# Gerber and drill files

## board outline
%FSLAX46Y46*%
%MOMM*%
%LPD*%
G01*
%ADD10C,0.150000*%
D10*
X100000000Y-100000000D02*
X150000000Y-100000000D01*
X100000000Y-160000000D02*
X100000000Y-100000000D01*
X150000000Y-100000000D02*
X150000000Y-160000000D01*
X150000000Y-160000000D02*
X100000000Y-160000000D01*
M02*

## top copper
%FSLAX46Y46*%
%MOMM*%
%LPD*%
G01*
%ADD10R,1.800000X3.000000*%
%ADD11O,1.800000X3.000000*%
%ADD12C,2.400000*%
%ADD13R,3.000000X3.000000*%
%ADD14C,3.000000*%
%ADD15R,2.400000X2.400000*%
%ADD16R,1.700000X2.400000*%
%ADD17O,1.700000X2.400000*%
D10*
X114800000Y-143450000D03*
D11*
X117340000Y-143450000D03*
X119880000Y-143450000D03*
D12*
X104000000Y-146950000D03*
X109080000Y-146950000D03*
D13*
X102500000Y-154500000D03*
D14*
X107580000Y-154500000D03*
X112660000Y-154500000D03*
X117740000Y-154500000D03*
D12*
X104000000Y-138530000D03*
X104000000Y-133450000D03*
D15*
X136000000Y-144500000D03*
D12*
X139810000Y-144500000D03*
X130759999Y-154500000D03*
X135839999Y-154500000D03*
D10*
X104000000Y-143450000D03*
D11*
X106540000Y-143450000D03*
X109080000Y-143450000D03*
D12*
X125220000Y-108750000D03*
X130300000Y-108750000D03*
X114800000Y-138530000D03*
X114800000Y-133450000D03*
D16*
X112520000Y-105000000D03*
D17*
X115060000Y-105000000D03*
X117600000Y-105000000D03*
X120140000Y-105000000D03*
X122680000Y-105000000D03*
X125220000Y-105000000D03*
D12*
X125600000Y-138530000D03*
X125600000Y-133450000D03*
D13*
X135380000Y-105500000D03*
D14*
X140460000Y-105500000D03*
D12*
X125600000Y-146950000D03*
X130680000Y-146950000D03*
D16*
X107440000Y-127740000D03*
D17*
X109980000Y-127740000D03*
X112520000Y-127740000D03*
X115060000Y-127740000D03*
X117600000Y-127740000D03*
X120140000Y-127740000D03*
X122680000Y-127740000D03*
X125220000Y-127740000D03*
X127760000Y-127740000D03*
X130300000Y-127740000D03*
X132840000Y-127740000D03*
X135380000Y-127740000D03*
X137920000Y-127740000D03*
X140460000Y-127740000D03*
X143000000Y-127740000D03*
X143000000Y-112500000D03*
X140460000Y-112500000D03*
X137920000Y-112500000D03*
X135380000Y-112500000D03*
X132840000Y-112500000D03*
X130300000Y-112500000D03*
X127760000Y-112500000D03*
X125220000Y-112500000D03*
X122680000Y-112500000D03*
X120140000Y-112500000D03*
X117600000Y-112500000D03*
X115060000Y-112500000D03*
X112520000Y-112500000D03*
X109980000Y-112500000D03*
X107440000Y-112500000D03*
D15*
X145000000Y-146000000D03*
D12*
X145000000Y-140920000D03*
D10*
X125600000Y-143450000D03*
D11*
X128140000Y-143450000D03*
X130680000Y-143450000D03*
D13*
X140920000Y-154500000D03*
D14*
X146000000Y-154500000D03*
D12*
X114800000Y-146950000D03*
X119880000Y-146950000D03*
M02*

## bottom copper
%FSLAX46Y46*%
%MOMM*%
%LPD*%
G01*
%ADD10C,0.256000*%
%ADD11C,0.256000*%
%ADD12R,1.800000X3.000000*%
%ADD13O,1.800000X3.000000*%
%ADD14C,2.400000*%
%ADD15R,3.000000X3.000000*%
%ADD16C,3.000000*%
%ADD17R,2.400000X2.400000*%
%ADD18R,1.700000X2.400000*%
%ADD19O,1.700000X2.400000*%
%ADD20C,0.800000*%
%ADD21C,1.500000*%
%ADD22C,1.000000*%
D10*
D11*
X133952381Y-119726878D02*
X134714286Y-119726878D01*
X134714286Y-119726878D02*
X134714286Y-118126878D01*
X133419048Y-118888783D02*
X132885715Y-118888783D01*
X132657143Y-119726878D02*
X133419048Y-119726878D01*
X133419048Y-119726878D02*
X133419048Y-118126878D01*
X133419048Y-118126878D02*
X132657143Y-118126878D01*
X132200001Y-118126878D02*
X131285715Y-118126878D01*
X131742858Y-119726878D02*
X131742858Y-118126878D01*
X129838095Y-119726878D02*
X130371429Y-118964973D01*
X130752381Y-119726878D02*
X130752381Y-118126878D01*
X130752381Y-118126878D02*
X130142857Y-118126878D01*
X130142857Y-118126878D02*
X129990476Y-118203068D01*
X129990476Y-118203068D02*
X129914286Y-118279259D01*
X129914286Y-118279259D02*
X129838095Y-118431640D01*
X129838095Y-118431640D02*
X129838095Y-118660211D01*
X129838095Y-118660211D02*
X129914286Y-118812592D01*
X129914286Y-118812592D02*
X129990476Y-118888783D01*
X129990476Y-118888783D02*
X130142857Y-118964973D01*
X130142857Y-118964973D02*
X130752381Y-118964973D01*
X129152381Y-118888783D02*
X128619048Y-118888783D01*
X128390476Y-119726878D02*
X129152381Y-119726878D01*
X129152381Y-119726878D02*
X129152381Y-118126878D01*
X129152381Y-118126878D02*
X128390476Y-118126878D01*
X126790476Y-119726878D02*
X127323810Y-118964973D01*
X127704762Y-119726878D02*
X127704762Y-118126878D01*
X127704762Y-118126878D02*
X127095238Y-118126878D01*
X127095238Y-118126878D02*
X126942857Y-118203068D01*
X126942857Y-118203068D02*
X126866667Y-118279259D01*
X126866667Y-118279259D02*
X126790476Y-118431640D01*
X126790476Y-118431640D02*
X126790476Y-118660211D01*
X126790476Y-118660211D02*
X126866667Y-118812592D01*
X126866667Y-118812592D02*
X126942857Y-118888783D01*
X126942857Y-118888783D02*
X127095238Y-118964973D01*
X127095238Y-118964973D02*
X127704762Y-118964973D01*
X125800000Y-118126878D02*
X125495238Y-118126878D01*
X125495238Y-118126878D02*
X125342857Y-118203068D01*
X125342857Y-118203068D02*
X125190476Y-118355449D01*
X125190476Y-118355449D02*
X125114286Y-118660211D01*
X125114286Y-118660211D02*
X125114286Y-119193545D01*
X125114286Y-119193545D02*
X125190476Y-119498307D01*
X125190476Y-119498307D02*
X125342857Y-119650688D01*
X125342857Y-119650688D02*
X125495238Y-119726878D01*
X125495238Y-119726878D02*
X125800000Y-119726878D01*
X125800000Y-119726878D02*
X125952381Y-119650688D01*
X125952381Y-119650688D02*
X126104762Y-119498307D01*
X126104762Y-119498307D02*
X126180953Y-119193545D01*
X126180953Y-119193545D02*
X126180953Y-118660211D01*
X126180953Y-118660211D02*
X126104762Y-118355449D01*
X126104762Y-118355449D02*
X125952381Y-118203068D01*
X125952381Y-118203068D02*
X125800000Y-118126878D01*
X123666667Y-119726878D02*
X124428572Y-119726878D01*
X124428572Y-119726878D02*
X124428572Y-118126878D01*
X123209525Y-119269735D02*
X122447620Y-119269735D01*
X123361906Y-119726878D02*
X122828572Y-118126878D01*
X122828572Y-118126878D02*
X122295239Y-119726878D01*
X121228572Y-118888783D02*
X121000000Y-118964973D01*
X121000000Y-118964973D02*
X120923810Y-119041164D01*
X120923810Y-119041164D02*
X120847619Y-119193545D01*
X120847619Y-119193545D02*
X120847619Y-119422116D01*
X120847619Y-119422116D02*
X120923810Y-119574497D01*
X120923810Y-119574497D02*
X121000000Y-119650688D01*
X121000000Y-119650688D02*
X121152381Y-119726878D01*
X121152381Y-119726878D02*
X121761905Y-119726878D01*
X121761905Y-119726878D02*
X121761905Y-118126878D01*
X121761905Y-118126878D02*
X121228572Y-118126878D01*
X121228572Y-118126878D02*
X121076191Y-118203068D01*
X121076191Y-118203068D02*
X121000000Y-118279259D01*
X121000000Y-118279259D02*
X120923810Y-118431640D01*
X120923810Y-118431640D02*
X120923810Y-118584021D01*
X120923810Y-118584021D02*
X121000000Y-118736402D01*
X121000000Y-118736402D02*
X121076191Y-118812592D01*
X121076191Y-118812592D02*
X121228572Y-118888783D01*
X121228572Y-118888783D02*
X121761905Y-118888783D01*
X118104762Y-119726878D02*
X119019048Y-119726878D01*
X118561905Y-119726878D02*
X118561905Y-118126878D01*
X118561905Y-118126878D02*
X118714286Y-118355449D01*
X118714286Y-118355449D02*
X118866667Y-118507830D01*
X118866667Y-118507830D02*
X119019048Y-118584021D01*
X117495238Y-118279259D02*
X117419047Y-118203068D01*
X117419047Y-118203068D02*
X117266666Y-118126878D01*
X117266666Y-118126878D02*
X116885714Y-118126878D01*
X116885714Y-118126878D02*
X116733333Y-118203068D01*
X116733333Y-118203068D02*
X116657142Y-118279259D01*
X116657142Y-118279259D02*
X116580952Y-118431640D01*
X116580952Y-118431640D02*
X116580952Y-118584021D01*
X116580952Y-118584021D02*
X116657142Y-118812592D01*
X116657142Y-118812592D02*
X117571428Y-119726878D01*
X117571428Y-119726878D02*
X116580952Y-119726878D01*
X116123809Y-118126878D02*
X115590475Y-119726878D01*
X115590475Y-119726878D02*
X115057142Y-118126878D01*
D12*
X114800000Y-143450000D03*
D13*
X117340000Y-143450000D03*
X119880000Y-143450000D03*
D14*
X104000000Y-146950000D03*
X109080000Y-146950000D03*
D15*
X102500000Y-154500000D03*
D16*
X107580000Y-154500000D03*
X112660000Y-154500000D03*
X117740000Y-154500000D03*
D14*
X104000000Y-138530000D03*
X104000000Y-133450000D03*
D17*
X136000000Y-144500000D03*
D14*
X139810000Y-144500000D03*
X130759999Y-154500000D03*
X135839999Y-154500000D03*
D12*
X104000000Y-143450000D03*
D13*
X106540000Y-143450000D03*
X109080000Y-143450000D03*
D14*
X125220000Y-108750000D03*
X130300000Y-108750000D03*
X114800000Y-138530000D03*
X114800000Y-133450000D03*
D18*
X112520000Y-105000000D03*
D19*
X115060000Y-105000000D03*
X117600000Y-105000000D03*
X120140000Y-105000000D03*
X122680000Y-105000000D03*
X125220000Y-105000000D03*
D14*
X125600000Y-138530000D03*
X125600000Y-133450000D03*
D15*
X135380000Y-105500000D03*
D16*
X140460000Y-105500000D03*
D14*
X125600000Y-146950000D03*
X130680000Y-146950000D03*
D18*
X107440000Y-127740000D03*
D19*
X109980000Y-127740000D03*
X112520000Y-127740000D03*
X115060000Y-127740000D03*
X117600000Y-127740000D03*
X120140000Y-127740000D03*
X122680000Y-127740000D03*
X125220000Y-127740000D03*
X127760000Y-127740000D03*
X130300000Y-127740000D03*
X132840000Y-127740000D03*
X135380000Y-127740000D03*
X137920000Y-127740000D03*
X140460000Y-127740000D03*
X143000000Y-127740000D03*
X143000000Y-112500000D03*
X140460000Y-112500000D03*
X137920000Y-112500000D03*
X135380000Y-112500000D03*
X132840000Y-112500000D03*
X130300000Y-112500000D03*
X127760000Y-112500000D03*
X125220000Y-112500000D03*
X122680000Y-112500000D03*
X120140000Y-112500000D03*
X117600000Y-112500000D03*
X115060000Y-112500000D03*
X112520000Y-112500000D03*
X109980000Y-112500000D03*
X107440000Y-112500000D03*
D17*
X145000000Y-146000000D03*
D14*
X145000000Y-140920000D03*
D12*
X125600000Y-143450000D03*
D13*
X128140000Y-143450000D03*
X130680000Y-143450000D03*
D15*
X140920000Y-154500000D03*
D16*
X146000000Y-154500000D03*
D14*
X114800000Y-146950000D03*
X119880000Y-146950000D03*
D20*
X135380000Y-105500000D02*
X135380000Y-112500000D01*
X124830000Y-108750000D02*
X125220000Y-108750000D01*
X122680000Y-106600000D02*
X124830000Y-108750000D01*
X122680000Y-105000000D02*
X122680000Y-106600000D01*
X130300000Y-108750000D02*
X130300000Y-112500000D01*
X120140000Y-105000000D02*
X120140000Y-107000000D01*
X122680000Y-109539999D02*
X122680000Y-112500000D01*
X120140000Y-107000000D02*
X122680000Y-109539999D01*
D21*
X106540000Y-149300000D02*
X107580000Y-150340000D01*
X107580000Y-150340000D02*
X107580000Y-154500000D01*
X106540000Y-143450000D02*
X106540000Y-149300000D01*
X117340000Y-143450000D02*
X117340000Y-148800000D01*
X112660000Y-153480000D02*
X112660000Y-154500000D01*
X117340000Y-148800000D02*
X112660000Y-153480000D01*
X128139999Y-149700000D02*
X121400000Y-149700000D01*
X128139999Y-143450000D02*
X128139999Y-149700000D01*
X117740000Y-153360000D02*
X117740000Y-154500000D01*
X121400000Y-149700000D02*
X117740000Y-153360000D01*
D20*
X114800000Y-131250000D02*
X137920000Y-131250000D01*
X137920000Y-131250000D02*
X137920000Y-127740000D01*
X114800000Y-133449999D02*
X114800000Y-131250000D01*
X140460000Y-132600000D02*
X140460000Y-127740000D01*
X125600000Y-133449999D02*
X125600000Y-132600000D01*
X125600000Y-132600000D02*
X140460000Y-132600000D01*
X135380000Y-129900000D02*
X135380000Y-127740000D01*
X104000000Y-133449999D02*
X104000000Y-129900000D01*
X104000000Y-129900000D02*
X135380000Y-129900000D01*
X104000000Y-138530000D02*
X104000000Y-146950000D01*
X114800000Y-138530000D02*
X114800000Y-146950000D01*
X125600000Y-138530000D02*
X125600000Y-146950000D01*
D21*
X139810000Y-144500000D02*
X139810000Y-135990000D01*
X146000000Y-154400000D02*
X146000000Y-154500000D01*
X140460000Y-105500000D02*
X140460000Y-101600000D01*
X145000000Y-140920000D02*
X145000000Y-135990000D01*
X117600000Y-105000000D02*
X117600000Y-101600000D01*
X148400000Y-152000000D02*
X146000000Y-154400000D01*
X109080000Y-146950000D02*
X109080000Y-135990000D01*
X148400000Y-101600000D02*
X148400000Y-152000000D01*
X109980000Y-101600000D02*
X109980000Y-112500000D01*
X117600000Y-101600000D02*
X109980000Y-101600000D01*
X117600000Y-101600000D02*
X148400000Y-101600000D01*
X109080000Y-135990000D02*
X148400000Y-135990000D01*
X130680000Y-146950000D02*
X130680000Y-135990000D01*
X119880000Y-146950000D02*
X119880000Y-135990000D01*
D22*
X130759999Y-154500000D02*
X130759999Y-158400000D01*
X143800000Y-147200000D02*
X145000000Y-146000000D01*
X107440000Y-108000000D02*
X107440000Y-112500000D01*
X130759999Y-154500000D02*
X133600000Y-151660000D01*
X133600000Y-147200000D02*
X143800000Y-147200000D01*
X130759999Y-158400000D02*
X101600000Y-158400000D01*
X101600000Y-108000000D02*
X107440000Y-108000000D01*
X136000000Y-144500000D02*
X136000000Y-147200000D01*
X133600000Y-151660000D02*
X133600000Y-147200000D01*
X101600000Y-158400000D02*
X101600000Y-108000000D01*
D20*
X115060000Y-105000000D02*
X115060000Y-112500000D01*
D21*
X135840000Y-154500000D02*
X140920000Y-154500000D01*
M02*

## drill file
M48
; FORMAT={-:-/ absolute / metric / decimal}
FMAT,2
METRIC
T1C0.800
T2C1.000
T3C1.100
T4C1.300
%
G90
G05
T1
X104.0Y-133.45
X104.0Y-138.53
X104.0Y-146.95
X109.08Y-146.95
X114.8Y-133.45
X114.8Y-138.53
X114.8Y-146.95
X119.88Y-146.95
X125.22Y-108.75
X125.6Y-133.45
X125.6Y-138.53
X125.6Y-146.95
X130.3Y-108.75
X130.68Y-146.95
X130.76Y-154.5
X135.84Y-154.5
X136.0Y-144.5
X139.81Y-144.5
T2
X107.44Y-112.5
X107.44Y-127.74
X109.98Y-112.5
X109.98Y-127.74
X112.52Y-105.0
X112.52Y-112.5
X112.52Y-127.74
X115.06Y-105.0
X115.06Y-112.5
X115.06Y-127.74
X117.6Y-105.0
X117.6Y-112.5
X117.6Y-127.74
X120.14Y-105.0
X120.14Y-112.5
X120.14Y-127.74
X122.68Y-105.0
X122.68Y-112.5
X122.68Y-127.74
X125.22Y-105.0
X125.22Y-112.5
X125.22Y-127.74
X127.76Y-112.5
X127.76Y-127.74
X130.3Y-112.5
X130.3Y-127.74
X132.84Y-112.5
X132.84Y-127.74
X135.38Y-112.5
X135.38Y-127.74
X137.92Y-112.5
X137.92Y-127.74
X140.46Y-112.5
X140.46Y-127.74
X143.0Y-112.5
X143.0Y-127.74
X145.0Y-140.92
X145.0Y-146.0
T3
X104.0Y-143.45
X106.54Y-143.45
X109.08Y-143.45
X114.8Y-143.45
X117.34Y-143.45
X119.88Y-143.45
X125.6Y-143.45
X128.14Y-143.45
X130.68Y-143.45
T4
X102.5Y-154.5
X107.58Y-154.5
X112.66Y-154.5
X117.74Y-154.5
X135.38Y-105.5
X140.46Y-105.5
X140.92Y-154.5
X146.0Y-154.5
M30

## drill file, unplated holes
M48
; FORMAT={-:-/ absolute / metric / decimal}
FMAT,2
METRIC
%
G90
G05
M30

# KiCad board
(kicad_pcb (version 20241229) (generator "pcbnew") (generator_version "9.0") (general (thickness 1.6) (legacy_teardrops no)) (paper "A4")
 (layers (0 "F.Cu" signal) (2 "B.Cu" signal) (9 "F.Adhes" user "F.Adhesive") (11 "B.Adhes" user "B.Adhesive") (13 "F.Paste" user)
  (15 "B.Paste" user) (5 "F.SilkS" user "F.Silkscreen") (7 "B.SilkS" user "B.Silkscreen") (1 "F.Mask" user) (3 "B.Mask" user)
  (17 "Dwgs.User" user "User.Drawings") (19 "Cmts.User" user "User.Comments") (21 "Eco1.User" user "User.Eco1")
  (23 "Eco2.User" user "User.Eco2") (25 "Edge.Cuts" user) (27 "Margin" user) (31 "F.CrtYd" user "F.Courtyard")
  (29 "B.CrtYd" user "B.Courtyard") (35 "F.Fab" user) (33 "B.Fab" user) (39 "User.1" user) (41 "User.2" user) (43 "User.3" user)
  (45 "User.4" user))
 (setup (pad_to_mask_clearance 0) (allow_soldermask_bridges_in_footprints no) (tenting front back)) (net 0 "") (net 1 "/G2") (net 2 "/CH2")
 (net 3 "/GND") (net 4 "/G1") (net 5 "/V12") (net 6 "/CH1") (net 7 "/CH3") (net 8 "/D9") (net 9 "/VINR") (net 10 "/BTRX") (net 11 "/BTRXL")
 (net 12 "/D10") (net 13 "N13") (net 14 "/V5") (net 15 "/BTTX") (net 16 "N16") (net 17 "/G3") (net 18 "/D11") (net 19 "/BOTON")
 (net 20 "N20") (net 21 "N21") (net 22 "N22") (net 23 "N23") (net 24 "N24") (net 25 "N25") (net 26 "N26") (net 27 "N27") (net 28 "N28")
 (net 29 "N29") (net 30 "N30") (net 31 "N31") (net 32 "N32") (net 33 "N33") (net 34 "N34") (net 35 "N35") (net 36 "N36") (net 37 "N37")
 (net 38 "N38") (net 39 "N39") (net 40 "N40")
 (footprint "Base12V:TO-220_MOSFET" (layer "F.Cu") (at 114.8 143.45)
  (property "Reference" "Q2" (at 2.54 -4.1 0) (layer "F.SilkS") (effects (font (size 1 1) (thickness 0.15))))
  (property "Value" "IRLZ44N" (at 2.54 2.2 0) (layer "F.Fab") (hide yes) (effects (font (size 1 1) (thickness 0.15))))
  (pad "1" thru_hole rect (at 0 0) (size 1.8 3) (drill 1.1) (layers "B.Cu" "B.Mask") (remove_unused_layers no) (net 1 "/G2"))
  (pad "2" thru_hole oval (at 2.54 0) (size 1.8 3) (drill 1.1) (layers "B.Cu" "B.Mask") (remove_unused_layers no) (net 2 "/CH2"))
  (pad "3" thru_hole oval (at 5.08 0) (size 1.8 3) (drill 1.1) (layers "B.Cu" "B.Mask") (remove_unused_layers no) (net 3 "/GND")))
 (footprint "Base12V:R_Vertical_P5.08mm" (layer "F.Cu") (at 104 146.95)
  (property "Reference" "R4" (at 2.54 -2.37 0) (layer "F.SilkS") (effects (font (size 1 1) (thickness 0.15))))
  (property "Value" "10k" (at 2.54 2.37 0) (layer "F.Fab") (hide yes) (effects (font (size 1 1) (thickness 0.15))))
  (pad "1" thru_hole circle (at 0 0) (size 2.4 2.4) (drill 0.8) (layers "B.Cu" "B.Mask") (remove_unused_layers no) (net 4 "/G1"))
  (pad "2" thru_hole circle (at 5.08 0) (size 2.4 2.4) (drill 0.8) (layers "B.Cu" "B.Mask") (remove_unused_layers no) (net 3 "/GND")))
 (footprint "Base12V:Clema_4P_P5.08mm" (layer "F.Cu") (at 102.5 154.5)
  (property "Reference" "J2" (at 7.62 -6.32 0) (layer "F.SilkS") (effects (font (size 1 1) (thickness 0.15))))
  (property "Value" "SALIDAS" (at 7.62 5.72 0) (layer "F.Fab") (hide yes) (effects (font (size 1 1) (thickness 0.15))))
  (pad "1" thru_hole rect (at 0 0) (size 3 3) (drill 1.3) (layers "B.Cu" "B.Mask") (remove_unused_layers no) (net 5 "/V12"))
  (pad "2" thru_hole circle (at 5.08 0) (size 3 3) (drill 1.3) (layers "B.Cu" "B.Mask") (remove_unused_layers no) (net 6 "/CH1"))
  (pad "3" thru_hole circle (at 10.16 0) (size 3 3) (drill 1.3) (layers "B.Cu" "B.Mask") (remove_unused_layers no) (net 2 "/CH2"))
  (pad "4" thru_hole circle (at 15.24 0) (size 3 3) (drill 1.3) (layers "B.Cu" "B.Mask") (remove_unused_layers no) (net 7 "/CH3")))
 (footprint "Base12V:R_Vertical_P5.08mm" (layer "F.Cu") (at 104 138.53 90)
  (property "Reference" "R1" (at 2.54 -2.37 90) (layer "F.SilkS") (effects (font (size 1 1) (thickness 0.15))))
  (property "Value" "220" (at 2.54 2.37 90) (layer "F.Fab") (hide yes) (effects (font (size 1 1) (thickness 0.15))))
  (pad "1" thru_hole circle (at 0 0 90) (size 2.4 2.4) (drill 0.8) (layers "B.Cu" "B.Mask") (remove_unused_layers no) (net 4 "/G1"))
  (pad "2" thru_hole circle (at 5.08 0 90) (size 2.4 2.4) (drill 0.8) (layers "B.Cu" "B.Mask") (remove_unused_layers no) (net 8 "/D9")))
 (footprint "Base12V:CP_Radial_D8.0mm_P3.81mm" (layer "F.Cu") (at 136 144.5)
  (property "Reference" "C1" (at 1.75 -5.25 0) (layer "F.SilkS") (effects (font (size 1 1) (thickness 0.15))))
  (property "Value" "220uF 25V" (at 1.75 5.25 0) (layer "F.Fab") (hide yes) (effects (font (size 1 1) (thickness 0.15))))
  (pad "1" thru_hole rect (at 0 0) (size 2.4 2.4) (drill 0.8) (layers "B.Cu" "B.Mask") (remove_unused_layers no) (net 5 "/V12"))
  (pad "2" thru_hole circle (at 3.81 0) (size 2.4 2.4) (drill 0.8) (layers "B.Cu" "B.Mask") (remove_unused_layers no) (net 3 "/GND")))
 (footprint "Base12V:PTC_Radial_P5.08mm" (layer "F.Cu") (at 130.759999 154.5)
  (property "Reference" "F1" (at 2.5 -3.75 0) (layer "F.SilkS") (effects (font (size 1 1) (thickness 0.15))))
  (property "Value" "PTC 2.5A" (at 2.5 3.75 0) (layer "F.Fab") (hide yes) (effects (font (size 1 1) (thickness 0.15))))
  (pad "1" thru_hole circle (at 0 0) (size 2.4 2.4) (drill 0.8) (layers "B.Cu" "B.Mask") (remove_unused_layers no) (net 5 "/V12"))
  (pad "2" thru_hole circle (at 5.08 0) (size 2.4 2.4) (drill 0.8) (layers "B.Cu" "B.Mask") (remove_unused_layers no) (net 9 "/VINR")))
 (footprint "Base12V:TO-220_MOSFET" (layer "F.Cu") (at 104 143.45)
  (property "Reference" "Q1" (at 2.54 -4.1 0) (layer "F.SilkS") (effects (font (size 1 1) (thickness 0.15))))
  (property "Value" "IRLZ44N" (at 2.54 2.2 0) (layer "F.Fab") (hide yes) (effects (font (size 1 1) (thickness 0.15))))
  (pad "1" thru_hole rect (at 0 0) (size 1.8 3) (drill 1.1) (layers "B.Cu" "B.Mask") (remove_unused_layers no) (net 4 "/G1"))
  (pad "2" thru_hole oval (at 2.54 0) (size 1.8 3) (drill 1.1) (layers "B.Cu" "B.Mask") (remove_unused_layers no) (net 6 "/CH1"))
  (pad "3" thru_hole oval (at 5.08 0) (size 1.8 3) (drill 1.1) (layers "B.Cu" "B.Mask") (remove_unused_layers no) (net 3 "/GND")))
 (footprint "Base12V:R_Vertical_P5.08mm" (layer "F.Cu") (at 125.22 108.75)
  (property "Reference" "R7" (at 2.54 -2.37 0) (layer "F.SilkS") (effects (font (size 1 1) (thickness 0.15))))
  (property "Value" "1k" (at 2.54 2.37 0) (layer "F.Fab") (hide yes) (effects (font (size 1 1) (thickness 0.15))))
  (pad "1" thru_hole circle (at 0 0) (size 2.4 2.4) (drill 0.8) (layers "B.Cu" "B.Mask") (remove_unused_layers no) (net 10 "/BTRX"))
  (pad "2" thru_hole circle (at 5.08 0) (size 2.4 2.4) (drill 0.8) (layers "B.Cu" "B.Mask") (remove_unused_layers no) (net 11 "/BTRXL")))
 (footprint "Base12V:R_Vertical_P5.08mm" (layer "F.Cu") (at 114.8 138.53 90)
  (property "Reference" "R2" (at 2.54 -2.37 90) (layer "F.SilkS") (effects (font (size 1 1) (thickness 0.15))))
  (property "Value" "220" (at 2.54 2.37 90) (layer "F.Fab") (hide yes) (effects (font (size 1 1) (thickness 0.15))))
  (pad "1" thru_hole circle (at 0 0 90) (size 2.4 2.4) (drill 0.8) (layers "B.Cu" "B.Mask") (remove_unused_layers no) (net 1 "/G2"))
  (pad "2" thru_hole circle (at 5.08 0 90) (size 2.4 2.4) (drill 0.8) (layers "B.Cu" "B.Mask") (remove_unused_layers no) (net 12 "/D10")))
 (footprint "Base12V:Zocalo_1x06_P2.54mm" (layer "F.Cu") (at 112.52 105 90)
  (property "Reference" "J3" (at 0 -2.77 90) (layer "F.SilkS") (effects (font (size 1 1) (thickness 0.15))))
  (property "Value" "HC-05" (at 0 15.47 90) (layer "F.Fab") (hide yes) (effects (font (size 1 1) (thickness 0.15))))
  (pad "1" thru_hole rect (at 0 0 90) (size 2.4 1.7) (drill 1) (layers "B.Cu" "B.Mask") (remove_unused_layers no) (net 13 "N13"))
  (pad "2" thru_hole oval (at 0 2.54 90) (size 2.4 1.7) (drill 1) (layers "B.Cu" "B.Mask") (remove_unused_layers no) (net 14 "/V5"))
  (pad "3" thru_hole oval (at 0 5.08 90) (size 2.4 1.7) (drill 1) (layers "B.Cu" "B.Mask") (remove_unused_layers no) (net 3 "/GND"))
  (pad "4" thru_hole oval (at 0 7.62 90) (size 2.4 1.7) (drill 1) (layers "B.Cu" "B.Mask") (remove_unused_layers no) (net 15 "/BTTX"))
  (pad "5" thru_hole oval (at 0 10.16 90) (size 2.4 1.7) (drill 1) (layers "B.Cu" "B.Mask") (remove_unused_layers no) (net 10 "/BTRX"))
  (pad "6" thru_hole oval (at 0 12.7 90) (size 2.4 1.7) (drill 1) (layers "B.Cu" "B.Mask") (remove_unused_layers no) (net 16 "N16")))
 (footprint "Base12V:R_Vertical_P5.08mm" (layer "F.Cu") (at 125.6 138.53 90)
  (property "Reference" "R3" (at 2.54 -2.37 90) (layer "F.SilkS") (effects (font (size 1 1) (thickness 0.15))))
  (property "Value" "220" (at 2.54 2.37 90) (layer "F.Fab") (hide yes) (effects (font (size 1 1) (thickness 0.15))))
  (pad "1" thru_hole circle (at 0 0 90) (size 2.4 2.4) (drill 0.8) (layers "B.Cu" "B.Mask") (remove_unused_layers no) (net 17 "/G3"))
  (pad "2" thru_hole circle (at 5.08 0 90) (size 2.4 2.4) (drill 0.8) (layers "B.Cu" "B.Mask") (remove_unused_layers no) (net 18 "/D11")))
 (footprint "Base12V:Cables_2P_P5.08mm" (layer "F.Cu") (at 135.38 105.5 90)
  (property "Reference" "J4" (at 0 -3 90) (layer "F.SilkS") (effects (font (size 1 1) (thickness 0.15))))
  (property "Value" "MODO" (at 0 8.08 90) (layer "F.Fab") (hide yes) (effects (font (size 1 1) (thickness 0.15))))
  (pad "1" thru_hole rect (at 0 0 90) (size 3 3) (drill 1.3) (layers "B.Cu" "B.Mask") (remove_unused_layers no) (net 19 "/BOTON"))
  (pad "2" thru_hole circle (at 0 5.08 90) (size 3 3) (drill 1.3) (layers "B.Cu" "B.Mask") (remove_unused_layers no) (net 3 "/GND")))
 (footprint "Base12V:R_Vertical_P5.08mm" (layer "F.Cu") (at 125.6 146.95)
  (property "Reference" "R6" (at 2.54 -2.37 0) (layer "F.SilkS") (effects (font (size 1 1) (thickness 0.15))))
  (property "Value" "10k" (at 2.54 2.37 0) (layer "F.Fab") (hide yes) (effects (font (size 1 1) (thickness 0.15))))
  (pad "1" thru_hole circle (at 0 0) (size 2.4 2.4) (drill 0.8) (layers "B.Cu" "B.Mask") (remove_unused_layers no) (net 17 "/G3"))
  (pad "2" thru_hole circle (at 5.08 0) (size 2.4 2.4) (drill 0.8) (layers "B.Cu" "B.Mask") (remove_unused_layers no) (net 3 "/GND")))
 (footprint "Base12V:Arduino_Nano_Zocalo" (layer "F.Cu") (at 107.44 127.74 90)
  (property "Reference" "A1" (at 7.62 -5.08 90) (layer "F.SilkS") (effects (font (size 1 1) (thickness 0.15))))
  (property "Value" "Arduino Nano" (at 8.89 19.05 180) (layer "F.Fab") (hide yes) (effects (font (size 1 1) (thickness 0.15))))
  (pad "1" thru_hole rect (at 0 0 90) (size 2.4 1.7) (drill 1) (layers "B.Cu" "B.Mask") (remove_unused_layers no) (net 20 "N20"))
  (pad "2" thru_hole oval (at 0 2.54 90) (size 2.4 1.7) (drill 1) (layers "B.Cu" "B.Mask") (remove_unused_layers no) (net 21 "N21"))
  (pad "3" thru_hole oval (at 0 5.08 90) (size 2.4 1.7) (drill 1) (layers "B.Cu" "B.Mask") (remove_unused_layers no) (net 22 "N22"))
  (pad "4" thru_hole oval (at 0 7.62 90) (size 2.4 1.7) (drill 1) (layers "B.Cu" "B.Mask") (remove_unused_layers no) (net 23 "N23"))
  (pad "5" thru_hole oval (at 0 10.16 90) (size 2.4 1.7) (drill 1) (layers "B.Cu" "B.Mask") (remove_unused_layers no) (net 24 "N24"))
  (pad "6" thru_hole oval (at 0 12.7 90) (size 2.4 1.7) (drill 1) (layers "B.Cu" "B.Mask") (remove_unused_layers no) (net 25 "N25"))
  (pad "7" thru_hole oval (at 0 15.24 90) (size 2.4 1.7) (drill 1) (layers "B.Cu" "B.Mask") (remove_unused_layers no) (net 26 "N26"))
  (pad "8" thru_hole oval (at 0 17.78 90) (size 2.4 1.7) (drill 1) (layers "B.Cu" "B.Mask") (remove_unused_layers no) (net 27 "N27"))
  (pad "9" thru_hole oval (at 0 20.32 90) (size 2.4 1.7) (drill 1) (layers "B.Cu" "B.Mask") (remove_unused_layers no) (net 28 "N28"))
  (pad "10" thru_hole oval (at 0 22.86 90) (size 2.4 1.7) (drill 1) (layers "B.Cu" "B.Mask") (remove_unused_layers no) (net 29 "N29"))
  (pad "11" thru_hole oval (at 0 25.4 90) (size 2.4 1.7) (drill 1) (layers "B.Cu" "B.Mask") (remove_unused_layers no) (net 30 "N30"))
  (pad "12" thru_hole oval (at 0 27.94 90) (size 2.4 1.7) (drill 1) (layers "B.Cu" "B.Mask") (remove_unused_layers no) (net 8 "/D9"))
  (pad "13" thru_hole oval (at 0 30.48 90) (size 2.4 1.7) (drill 1) (layers "B.Cu" "B.Mask") (remove_unused_layers no) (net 12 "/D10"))
  (pad "14" thru_hole oval (at 0 33.02 90) (size 2.4 1.7) (drill 1) (layers "B.Cu" "B.Mask") (remove_unused_layers no) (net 18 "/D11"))
  (pad "15" thru_hole oval (at 0 35.56 90) (size 2.4 1.7) (drill 1) (layers "B.Cu" "B.Mask") (remove_unused_layers no) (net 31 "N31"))
  (pad "16" thru_hole oval (at 15.24 35.56 90) (size 2.4 1.7) (drill 1) (layers "B.Cu" "B.Mask") (remove_unused_layers no) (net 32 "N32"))
  (pad "17" thru_hole oval (at 15.24 33.02 90) (size 2.4 1.7) (drill 1) (layers "B.Cu" "B.Mask") (remove_unused_layers no) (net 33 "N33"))
  (pad "18" thru_hole oval (at 15.24 30.48 90) (size 2.4 1.7) (drill 1) (layers "B.Cu" "B.Mask") (remove_unused_layers no) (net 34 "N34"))
  (pad "19" thru_hole oval (at 15.24 27.94 90) (size 2.4 1.7) (drill 1) (layers "B.Cu" "B.Mask") (remove_unused_layers no) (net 19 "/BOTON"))
  (pad "20" thru_hole oval (at 15.24 25.4 90) (size 2.4 1.7) (drill 1) (layers "B.Cu" "B.Mask") (remove_unused_layers no) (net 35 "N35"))
  (pad "21" thru_hole oval (at 15.24 22.86 90) (size 2.4 1.7) (drill 1) (layers "B.Cu" "B.Mask") (remove_unused_layers no) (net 11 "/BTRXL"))
  (pad "22" thru_hole oval (at 15.24 20.32 90) (size 2.4 1.7) (drill 1) (layers "B.Cu" "B.Mask") (remove_unused_layers no) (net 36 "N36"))
  (pad "23" thru_hole oval (at 15.24 17.78 90) (size 2.4 1.7) (drill 1) (layers "B.Cu" "B.Mask") (remove_unused_layers no) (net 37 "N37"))
  (pad "24" thru_hole oval (at 15.24 15.24 90) (size 2.4 1.7) (drill 1) (layers "B.Cu" "B.Mask") (remove_unused_layers no) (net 15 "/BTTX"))
  (pad "25" thru_hole oval (at 15.24 12.7 90) (size 2.4 1.7) (drill 1) (layers "B.Cu" "B.Mask") (remove_unused_layers no) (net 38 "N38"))
  (pad "26" thru_hole oval (at 15.24 10.16 90) (size 2.4 1.7) (drill 1) (layers "B.Cu" "B.Mask") (remove_unused_layers no) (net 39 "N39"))
  (pad "27" thru_hole oval (at 15.24 7.62 90) (size 2.4 1.7) (drill 1) (layers "B.Cu" "B.Mask") (remove_unused_layers no) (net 14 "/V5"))
  (pad "28" thru_hole oval (at 15.24 5.08 90) (size 2.4 1.7) (drill 1) (layers "B.Cu" "B.Mask") (remove_unused_layers no) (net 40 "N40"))
  (pad "29" thru_hole oval (at 15.24 2.54 90) (size 2.4 1.7) (drill 1) (layers "B.Cu" "B.Mask") (remove_unused_layers no) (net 3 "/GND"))
  (pad "30" thru_hole oval (at 15.24 0 90) (size 2.4 1.7) (drill 1) (layers "B.Cu" "B.Mask") (remove_unused_layers no) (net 5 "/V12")))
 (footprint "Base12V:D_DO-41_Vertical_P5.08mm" (layer "F.Cu") (at 145 146 90)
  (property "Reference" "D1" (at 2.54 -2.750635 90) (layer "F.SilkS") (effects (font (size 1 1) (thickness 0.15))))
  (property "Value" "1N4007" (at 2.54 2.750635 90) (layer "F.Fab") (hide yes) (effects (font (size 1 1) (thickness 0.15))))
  (pad "1" thru_hole rect (at 0 0 90) (size 2.4 2.4) (drill 1) (layers "B.Cu" "B.Mask") (remove_unused_layers no) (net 5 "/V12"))
  (pad "2" thru_hole circle (at 5.08 0 90) (size 2.4 2.4) (drill 1) (layers "B.Cu" "B.Mask") (remove_unused_layers no) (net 3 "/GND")))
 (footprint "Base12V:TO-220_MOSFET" (layer "F.Cu") (at 125.6 143.45)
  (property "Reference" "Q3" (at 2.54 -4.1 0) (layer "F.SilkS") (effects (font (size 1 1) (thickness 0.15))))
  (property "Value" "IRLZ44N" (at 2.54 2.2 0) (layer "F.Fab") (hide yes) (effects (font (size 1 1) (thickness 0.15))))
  (pad "1" thru_hole rect (at 0 0) (size 1.8 3) (drill 1.1) (layers "B.Cu" "B.Mask") (remove_unused_layers no) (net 17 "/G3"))
  (pad "2" thru_hole oval (at 2.54 0) (size 1.8 3) (drill 1.1) (layers "B.Cu" "B.Mask") (remove_unused_layers no) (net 7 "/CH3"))
  (pad "3" thru_hole oval (at 5.08 0) (size 1.8 3) (drill 1.1) (layers "B.Cu" "B.Mask") (remove_unused_layers no) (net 3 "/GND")))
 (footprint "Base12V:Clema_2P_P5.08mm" (layer "F.Cu") (at 140.92 154.5)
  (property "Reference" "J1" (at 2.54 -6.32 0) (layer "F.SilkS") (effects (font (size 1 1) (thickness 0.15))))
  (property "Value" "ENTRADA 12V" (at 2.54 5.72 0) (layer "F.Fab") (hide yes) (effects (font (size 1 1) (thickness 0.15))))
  (pad "1" thru_hole rect (at 0 0) (size 3 3) (drill 1.3) (layers "B.Cu" "B.Mask") (remove_unused_layers no) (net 9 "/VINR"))
  (pad "2" thru_hole circle (at 5.08 0) (size 3 3) (drill 1.3) (layers "B.Cu" "B.Mask") (remove_unused_layers no) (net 3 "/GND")))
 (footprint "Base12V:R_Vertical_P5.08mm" (layer "F.Cu") (at 114.8 146.95)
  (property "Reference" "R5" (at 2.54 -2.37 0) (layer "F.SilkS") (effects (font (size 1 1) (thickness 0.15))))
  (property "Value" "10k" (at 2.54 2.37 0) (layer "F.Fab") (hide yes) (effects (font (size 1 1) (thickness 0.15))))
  (pad "1" thru_hole circle (at 0 0) (size 2.4 2.4) (drill 0.8) (layers "B.Cu" "B.Mask") (remove_unused_layers no) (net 1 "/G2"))
  (pad "2" thru_hole circle (at 5.08 0) (size 2.4 2.4) (drill 0.8) (layers "B.Cu" "B.Mask") (remove_unused_layers no) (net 3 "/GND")))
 (gr_line (start 100 100) (end 150 100) (stroke (width 0.15) (type default)) (layer "Edge.Cuts"))
 (gr_line (start 100 160) (end 100 100) (stroke (width 0.15) (type default)) (layer "Edge.Cuts"))
 (gr_line (start 150 100) (end 150 160) (stroke (width 0.15) (type default)) (layer "Edge.Cuts"))
 (gr_line (start 150 160) (end 100 160) (stroke (width 0.15) (type default)) (layer "Edge.Cuts"))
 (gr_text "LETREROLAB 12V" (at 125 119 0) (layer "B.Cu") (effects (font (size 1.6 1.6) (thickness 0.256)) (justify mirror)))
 (segment (start 135.38 105.5) (end 135.38 112.5) (width 0.8) (layer "B.Cu") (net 19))
 (segment (start 124.83 108.75) (end 125.22 108.75) (width 0.8) (layer "B.Cu") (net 10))
 (segment (start 122.68 106.6) (end 124.83 108.75) (width 0.8) (layer "B.Cu") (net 10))
 (segment (start 122.68 105) (end 122.68 106.6) (width 0.8) (layer "B.Cu") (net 10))
 (segment (start 130.3 108.75) (end 130.3 112.5) (width 0.8) (layer "B.Cu") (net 11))
 (segment (start 120.14 105) (end 120.14 107) (width 0.8) (layer "B.Cu") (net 15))
 (segment (start 122.68 109.539999) (end 122.68 112.5) (width 0.8) (layer "B.Cu") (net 15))
 (segment (start 120.14 107) (end 122.68 109.539999) (width 0.8) (layer "B.Cu") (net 15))
 (segment (start 106.54 149.3) (end 107.58 150.34) (width 1.5) (layer "B.Cu") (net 6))
 (segment (start 107.58 150.34) (end 107.58 154.5) (width 1.5) (layer "B.Cu") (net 6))
 (segment (start 106.54 143.45) (end 106.54 149.3) (width 1.5) (layer "B.Cu") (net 6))
 (segment (start 117.34 143.45) (end 117.34 148.8) (width 1.5) (layer "B.Cu") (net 2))
 (segment (start 112.66 153.48) (end 112.66 154.5) (width 1.5) (layer "B.Cu") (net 2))
 (segment (start 117.34 148.8) (end 112.66 153.48) (width 1.5) (layer "B.Cu") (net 2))
 (segment (start 128.139999 149.7) (end 121.4 149.7) (width 1.5) (layer "B.Cu") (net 7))
 (segment (start 128.139999 143.45) (end 128.139999 149.7) (width 1.5) (layer "B.Cu") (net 7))
 (segment (start 117.74 153.36) (end 117.74 154.5) (width 1.5) (layer "B.Cu") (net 7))
 (segment (start 121.4 149.7) (end 117.74 153.36) (width 1.5) (layer "B.Cu") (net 7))
 (segment (start 114.8 131.25) (end 137.92 131.25) (width 0.8) (layer "B.Cu") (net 12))
 (segment (start 137.92 131.25) (end 137.92 127.74) (width 0.8) (layer "B.Cu") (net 12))
 (segment (start 114.8 133.449999) (end 114.8 131.25) (width 0.8) (layer "B.Cu") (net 12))
 (segment (start 140.46 132.6) (end 140.46 127.74) (width 0.8) (layer "B.Cu") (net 18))
 (segment (start 125.6 133.449999) (end 125.6 132.6) (width 0.8) (layer "B.Cu") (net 18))
 (segment (start 125.6 132.6) (end 140.46 132.6) (width 0.8) (layer "B.Cu") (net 18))
 (segment (start 135.38 129.9) (end 135.38 127.74) (width 0.8) (layer "B.Cu") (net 8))
 (segment (start 104 133.449999) (end 104 129.9) (width 0.8) (layer "B.Cu") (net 8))
 (segment (start 104 129.9) (end 135.38 129.9) (width 0.8) (layer "B.Cu") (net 8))
 (segment (start 104 138.53) (end 104 146.95) (width 0.8) (layer "B.Cu") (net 4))
 (segment (start 114.8 138.53) (end 114.8 146.95) (width 0.8) (layer "B.Cu") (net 1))
 (segment (start 125.6 138.53) (end 125.6 146.95) (width 0.8) (layer "B.Cu") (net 17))
 (segment (start 139.81 144.5) (end 139.81 135.99) (width 1.5) (layer "B.Cu") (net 3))
 (segment (start 146 154.4) (end 146 154.5) (width 1.5) (layer "B.Cu") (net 3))
 (segment (start 140.46 105.5) (end 140.46 101.6) (width 1.5) (layer "B.Cu") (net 3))
 (segment (start 145 140.92) (end 145 135.99) (width 1.5) (layer "B.Cu") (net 3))
 (segment (start 117.6 105) (end 117.6 101.6) (width 1.5) (layer "B.Cu") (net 3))
 (segment (start 148.4 152) (end 146 154.4) (width 1.5) (layer "B.Cu") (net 3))
 (segment (start 109.08 146.95) (end 109.08 135.99) (width 1.5) (layer "B.Cu") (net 3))
 (segment (start 148.4 101.6) (end 148.4 152) (width 1.5) (layer "B.Cu") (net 3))
 (segment (start 109.98 101.6) (end 109.98 112.5) (width 1.5) (layer "B.Cu") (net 3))
 (segment (start 117.6 101.6) (end 109.98 101.6) (width 1.5) (layer "B.Cu") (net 3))
 (segment (start 117.6 101.6) (end 148.4 101.6) (width 1.5) (layer "B.Cu") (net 3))
 (segment (start 109.08 135.99) (end 148.4 135.99) (width 1.5) (layer "B.Cu") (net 3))
 (segment (start 130.68 146.95) (end 130.68 135.99) (width 1.5) (layer "B.Cu") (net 3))
 (segment (start 119.88 146.95) (end 119.88 135.99) (width 1.5) (layer "B.Cu") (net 3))
 (segment (start 130.759999 154.5) (end 130.759999 158.4) (width 1) (layer "B.Cu") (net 5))
 (segment (start 143.8 147.2) (end 145 146) (width 1) (layer "B.Cu") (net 5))
 (segment (start 107.44 108) (end 107.44 112.5) (width 1) (layer "B.Cu") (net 5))
 (segment (start 130.759999 154.5) (end 133.6 151.66) (width 1) (layer "B.Cu") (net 5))
 (segment (start 133.6 147.2) (end 143.8 147.2) (width 1) (layer "B.Cu") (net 5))
 (segment (start 130.759999 158.4) (end 101.6 158.4) (width 1) (layer "B.Cu") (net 5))
 (segment (start 101.6 108) (end 107.44 108) (width 1) (layer "B.Cu") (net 5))
 (segment (start 136 144.5) (end 136 147.2) (width 1) (layer "B.Cu") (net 5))
 (segment (start 133.6 151.66) (end 133.6 147.2) (width 1) (layer "B.Cu") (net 5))
 (segment (start 101.6 158.4) (end 101.6 108) (width 1) (layer "B.Cu") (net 5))
 (segment (start 115.06 105) (end 115.06 112.5) (width 0.8) (layer "B.Cu") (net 14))
 (segment (start 135.84 154.5) (end 140.92 154.5) (width 1.5) (layer "B.Cu") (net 9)))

